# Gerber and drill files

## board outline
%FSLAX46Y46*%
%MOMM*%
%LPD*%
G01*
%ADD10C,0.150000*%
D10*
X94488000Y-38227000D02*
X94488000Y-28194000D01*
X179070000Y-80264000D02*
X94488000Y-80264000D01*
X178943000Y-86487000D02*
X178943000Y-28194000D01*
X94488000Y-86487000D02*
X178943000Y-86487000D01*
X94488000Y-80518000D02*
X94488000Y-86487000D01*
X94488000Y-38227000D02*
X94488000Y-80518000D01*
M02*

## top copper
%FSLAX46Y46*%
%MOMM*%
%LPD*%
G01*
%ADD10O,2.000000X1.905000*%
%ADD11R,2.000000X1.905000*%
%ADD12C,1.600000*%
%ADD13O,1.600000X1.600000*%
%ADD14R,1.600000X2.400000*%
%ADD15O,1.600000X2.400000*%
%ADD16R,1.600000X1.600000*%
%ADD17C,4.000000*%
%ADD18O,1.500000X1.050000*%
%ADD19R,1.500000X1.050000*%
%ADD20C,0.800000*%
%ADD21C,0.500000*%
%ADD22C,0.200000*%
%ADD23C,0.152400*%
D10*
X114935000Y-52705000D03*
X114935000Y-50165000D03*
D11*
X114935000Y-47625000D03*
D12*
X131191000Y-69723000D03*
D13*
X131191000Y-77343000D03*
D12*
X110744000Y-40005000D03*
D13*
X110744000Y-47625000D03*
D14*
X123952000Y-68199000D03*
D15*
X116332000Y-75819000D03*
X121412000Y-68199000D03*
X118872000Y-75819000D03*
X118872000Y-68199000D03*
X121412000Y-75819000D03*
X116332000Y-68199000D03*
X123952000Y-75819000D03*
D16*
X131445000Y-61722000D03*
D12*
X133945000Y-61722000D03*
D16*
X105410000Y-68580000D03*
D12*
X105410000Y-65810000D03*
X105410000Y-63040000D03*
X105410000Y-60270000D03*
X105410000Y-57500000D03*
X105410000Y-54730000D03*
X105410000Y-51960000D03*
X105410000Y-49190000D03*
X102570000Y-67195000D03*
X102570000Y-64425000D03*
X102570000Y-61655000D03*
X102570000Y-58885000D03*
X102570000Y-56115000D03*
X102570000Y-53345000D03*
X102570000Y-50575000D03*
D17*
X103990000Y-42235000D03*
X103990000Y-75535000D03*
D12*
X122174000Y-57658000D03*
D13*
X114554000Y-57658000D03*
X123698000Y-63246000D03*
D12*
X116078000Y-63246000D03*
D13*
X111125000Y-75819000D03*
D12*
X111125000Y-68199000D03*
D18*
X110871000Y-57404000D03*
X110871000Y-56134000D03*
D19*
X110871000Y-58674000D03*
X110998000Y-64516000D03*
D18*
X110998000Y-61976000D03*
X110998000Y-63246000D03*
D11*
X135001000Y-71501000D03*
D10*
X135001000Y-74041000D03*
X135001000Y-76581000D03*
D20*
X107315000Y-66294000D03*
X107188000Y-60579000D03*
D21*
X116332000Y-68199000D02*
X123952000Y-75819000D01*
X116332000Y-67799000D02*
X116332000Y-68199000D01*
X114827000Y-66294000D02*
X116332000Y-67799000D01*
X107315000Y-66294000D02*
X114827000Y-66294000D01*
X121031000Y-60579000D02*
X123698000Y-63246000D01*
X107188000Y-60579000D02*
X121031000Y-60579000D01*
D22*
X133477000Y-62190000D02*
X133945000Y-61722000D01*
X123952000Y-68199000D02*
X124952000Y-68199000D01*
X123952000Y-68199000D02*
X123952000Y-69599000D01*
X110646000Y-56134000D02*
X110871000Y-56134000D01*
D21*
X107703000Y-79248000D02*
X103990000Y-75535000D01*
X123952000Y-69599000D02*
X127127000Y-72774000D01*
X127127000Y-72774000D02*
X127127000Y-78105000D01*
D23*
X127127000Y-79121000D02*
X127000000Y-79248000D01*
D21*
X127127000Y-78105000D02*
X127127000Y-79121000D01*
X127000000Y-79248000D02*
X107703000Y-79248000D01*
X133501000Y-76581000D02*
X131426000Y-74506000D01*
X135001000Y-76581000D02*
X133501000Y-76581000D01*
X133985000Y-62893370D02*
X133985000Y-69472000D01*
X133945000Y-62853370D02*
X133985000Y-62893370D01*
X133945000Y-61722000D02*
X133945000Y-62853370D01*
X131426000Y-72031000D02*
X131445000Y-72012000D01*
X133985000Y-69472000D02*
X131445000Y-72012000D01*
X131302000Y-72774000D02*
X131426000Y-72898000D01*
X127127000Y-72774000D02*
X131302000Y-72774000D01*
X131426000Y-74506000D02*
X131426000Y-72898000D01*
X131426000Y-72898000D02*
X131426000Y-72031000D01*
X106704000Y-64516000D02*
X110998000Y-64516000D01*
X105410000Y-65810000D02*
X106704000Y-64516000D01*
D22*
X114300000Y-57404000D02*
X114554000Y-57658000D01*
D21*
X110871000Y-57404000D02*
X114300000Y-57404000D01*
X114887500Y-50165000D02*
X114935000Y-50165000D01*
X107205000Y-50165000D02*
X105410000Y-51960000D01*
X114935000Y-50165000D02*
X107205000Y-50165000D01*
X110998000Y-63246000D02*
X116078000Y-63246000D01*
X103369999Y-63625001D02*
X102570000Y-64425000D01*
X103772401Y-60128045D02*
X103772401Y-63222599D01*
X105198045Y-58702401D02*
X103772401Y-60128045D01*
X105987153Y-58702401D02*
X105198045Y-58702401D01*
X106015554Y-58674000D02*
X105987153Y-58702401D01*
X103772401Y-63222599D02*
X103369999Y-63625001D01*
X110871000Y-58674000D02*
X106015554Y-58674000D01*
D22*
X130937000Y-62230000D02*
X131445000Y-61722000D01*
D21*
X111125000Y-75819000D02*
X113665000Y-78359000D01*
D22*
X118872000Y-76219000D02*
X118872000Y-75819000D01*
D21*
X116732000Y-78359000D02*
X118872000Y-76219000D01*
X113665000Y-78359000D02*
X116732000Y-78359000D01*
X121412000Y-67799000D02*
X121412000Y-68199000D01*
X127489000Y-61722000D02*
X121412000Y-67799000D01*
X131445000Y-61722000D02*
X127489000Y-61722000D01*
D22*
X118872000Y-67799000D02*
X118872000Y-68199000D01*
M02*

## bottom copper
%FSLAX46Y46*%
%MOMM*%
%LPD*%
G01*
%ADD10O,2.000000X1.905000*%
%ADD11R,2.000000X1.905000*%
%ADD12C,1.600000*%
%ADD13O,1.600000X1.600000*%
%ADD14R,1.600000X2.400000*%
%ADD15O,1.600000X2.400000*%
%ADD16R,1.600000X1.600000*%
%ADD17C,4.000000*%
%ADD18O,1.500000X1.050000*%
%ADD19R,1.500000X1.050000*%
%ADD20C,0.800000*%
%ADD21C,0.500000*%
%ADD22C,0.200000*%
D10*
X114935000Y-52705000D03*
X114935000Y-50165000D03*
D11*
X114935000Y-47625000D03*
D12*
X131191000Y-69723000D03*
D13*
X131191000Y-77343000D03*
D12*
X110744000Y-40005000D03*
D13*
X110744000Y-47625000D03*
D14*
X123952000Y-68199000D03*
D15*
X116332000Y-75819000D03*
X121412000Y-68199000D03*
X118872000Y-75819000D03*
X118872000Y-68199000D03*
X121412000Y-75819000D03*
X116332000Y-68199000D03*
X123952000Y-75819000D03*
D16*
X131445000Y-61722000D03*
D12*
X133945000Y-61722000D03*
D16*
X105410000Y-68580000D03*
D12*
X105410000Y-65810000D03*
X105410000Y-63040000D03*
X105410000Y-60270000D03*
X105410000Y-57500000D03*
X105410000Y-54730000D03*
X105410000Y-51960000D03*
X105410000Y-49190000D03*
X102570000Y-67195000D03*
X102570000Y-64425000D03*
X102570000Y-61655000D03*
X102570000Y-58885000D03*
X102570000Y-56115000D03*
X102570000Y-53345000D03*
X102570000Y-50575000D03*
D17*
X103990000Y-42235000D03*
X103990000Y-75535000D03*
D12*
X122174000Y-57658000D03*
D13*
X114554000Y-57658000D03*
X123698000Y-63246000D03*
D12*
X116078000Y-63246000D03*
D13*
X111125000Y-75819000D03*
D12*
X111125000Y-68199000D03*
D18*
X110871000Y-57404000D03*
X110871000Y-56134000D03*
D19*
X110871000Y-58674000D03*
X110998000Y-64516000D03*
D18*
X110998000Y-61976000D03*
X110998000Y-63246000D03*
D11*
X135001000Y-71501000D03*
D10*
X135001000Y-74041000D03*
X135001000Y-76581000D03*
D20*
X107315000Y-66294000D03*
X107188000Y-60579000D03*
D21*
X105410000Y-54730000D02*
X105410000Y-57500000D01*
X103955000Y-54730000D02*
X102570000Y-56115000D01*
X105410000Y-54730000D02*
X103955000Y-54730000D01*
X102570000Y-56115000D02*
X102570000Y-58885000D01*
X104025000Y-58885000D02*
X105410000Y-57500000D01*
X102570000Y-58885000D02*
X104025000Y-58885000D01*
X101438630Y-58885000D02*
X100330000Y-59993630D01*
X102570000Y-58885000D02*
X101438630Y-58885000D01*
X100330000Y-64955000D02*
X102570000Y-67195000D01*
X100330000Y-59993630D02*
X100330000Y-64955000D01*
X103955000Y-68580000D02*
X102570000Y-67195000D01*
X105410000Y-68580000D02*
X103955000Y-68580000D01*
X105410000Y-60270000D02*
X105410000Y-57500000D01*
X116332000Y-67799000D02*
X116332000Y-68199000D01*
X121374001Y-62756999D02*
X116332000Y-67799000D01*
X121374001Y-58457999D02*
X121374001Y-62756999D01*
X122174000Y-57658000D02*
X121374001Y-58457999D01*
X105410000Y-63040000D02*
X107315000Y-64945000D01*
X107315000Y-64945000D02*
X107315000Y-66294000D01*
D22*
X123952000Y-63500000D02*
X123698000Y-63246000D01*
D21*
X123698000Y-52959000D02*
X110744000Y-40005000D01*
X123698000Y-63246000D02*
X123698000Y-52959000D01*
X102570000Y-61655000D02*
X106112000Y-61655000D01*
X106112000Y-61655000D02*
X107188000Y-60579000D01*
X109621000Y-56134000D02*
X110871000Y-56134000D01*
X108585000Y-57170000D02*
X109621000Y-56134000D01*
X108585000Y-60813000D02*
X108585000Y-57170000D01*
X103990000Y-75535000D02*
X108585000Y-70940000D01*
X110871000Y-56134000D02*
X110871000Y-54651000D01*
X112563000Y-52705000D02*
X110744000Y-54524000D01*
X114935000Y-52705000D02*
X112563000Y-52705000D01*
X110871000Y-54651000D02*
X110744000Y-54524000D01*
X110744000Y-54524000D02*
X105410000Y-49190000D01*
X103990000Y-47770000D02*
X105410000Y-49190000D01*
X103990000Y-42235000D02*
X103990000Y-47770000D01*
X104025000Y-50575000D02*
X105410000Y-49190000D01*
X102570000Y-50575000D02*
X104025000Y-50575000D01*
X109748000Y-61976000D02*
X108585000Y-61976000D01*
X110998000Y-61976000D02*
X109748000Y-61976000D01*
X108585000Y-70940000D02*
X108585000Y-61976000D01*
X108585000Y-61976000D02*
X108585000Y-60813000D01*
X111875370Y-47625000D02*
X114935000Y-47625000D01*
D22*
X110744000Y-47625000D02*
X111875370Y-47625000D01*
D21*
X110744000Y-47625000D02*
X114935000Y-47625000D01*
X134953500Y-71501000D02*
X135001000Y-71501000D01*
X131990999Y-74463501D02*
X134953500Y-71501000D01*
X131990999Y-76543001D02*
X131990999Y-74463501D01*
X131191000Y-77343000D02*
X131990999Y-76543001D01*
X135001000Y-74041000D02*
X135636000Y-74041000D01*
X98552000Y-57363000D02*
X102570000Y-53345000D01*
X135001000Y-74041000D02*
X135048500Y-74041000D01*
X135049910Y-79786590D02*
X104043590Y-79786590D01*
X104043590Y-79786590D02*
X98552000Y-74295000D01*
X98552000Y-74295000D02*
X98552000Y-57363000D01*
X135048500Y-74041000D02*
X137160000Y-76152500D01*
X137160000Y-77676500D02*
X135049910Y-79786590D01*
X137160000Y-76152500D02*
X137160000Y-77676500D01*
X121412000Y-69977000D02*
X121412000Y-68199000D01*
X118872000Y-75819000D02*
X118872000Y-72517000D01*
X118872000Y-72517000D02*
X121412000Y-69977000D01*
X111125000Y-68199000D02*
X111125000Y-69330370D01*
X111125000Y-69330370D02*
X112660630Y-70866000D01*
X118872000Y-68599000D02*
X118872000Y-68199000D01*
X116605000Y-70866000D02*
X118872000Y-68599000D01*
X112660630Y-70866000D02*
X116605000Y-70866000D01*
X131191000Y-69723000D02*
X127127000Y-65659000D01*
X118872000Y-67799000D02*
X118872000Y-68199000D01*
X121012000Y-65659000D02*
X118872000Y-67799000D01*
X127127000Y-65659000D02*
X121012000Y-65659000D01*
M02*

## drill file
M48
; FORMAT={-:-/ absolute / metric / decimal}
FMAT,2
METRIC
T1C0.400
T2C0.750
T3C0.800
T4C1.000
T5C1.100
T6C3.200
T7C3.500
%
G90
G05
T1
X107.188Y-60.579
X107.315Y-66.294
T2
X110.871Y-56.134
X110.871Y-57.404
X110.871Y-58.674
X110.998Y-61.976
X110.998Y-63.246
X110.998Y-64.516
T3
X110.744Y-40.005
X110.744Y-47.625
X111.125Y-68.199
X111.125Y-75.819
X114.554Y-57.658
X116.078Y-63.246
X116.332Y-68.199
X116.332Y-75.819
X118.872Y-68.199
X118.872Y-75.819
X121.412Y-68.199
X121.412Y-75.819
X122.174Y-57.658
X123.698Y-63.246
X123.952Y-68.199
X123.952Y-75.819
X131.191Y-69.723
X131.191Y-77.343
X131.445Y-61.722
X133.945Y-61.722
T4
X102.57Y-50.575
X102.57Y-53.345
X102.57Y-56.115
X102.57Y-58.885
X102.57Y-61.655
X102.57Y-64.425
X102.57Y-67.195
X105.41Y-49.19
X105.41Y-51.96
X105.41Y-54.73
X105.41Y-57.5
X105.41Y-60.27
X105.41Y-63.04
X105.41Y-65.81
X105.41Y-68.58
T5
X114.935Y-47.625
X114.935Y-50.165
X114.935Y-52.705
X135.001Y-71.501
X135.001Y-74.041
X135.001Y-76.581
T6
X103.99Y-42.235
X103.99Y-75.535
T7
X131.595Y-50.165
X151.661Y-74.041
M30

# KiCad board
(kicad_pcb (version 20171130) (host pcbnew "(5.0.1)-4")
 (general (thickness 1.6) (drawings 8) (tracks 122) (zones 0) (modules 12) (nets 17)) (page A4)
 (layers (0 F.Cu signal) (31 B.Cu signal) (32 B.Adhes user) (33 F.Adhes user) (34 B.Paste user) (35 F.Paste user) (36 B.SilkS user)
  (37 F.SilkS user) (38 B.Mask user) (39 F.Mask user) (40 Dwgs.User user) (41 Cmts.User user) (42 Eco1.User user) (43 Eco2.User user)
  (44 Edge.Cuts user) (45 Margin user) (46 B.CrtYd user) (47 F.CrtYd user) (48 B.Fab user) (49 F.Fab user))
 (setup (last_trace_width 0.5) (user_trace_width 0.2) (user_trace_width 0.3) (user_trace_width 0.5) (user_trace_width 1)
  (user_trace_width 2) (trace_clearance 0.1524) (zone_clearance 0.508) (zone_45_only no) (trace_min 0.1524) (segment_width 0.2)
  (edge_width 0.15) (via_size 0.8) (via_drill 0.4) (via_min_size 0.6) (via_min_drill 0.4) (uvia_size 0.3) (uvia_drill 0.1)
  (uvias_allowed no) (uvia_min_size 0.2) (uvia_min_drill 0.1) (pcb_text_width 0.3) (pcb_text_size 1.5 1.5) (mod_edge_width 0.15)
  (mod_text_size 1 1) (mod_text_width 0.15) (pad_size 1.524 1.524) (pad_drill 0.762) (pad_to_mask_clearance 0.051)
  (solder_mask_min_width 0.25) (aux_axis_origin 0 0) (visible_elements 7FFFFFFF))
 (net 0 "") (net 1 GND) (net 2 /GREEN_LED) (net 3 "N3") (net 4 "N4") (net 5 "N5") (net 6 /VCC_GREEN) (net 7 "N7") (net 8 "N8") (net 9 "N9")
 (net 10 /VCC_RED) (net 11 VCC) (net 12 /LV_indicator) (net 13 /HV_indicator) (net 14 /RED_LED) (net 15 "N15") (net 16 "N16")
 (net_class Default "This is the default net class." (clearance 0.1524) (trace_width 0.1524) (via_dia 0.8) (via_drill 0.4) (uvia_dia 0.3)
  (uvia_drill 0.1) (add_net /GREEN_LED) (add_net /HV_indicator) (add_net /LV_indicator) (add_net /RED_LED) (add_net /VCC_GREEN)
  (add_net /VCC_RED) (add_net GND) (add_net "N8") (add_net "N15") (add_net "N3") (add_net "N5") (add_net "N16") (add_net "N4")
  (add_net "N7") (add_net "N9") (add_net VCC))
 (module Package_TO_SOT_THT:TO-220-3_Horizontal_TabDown (layer F.Cu) (at 114.935 47.625 270)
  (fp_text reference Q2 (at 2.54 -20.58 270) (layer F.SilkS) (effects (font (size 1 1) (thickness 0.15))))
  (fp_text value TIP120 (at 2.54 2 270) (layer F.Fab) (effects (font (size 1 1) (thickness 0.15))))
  (pad 3 thru_hole oval (at 5.08 0 270) (size 1.905 2) (drill 1.1) (layers *.Cu *.Mask) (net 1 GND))
  (pad 2 thru_hole oval (at 2.54 0 270) (size 1.905 2) (drill 1.1) (layers *.Cu *.Mask) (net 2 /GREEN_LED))
  (pad 1 thru_hole rect (at 0 0 270) (size 1.905 2) (drill 1.1) (layers *.Cu *.Mask) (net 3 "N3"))
  (pad "" np_thru_hole oval (at 2.54 -16.66 270) (size 3.5 3.5) (drill 3.5) (layers *.Cu *.Mask)))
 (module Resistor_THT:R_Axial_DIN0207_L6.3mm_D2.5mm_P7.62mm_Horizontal (layer F.Cu) (at 131.191 69.723 270)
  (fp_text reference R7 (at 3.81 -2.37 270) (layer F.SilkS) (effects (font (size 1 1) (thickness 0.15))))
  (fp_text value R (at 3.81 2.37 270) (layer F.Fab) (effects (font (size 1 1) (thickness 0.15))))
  (pad 1 thru_hole circle (at 0 0 270) (size 1.6 1.6) (drill 0.8) (layers *.Cu *.Mask) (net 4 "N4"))
  (pad 2 thru_hole oval (at 7.62 0 270) (size 1.6 1.6) (drill 0.8) (layers *.Cu *.Mask) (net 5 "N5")))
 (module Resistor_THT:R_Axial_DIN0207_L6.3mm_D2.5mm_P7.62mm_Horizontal (layer F.Cu) (at 110.744 40.005 270)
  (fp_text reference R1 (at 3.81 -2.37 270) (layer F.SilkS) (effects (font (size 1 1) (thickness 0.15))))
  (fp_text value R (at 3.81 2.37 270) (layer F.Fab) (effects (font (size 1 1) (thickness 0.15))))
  (pad 1 thru_hole circle (at 0 0 270) (size 1.6 1.6) (drill 0.8) (layers *.Cu *.Mask) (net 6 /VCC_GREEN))
  (pad 2 thru_hole oval (at 7.62 0 270) (size 1.6 1.6) (drill 0.8) (layers *.Cu *.Mask) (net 3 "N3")))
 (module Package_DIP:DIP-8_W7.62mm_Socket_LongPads (layer F.Cu) (at 123.952 68.199 270)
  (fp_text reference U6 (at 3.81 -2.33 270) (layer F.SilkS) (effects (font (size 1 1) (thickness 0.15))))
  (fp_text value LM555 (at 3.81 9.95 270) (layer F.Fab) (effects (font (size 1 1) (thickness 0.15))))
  (pad 1 thru_hole rect (at 0 0 270) (size 2.4 1.6) (drill 0.8) (layers *.Cu *.Mask) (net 1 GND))
  (pad 5 thru_hole oval (at 7.62 7.62 270) (size 2.4 1.6) (drill 0.8) (layers *.Cu *.Mask) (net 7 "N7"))
  (pad 2 thru_hole oval (at 0 2.54 270) (size 2.4 1.6) (drill 0.8) (layers *.Cu *.Mask) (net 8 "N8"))
  (pad 6 thru_hole oval (at 7.62 5.08 270) (size 2.4 1.6) (drill 0.8) (layers *.Cu *.Mask) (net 8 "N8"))
  (pad 3 thru_hole oval (at 0 5.08 270) (size 2.4 1.6) (drill 0.8) (layers *.Cu *.Mask) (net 4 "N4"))
  (pad 7 thru_hole oval (at 7.62 2.54 270) (size 2.4 1.6) (drill 0.8) (layers *.Cu *.Mask) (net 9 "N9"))
  (pad 4 thru_hole oval (at 0 7.62 270) (size 2.4 1.6) (drill 0.8) (layers *.Cu *.Mask) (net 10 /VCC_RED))
  (pad 8 thru_hole oval (at 7.62 0 270) (size 2.4 1.6) (drill 0.8) (layers *.Cu *.Mask) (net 10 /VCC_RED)))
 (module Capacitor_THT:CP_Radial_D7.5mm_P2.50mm (layer F.Cu) (at 131.445 61.722)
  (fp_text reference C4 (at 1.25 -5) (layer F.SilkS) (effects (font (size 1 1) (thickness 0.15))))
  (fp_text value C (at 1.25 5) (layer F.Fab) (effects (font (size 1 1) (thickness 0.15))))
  (pad 1 thru_hole rect (at 0 0) (size 1.6 1.6) (drill 0.8) (layers *.Cu *.Mask) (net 8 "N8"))
  (pad 2 thru_hole circle (at 2.5 0) (size 1.6 1.6) (drill 0.8) (layers *.Cu *.Mask) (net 1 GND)))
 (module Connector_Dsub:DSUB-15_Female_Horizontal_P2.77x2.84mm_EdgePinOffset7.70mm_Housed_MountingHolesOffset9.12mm (layer F.Cu)
  (at 105.41 68.58 270)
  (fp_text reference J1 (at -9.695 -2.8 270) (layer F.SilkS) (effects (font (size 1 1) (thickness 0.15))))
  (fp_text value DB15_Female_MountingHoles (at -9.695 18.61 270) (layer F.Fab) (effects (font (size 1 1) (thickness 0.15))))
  (pad 1 thru_hole rect (at 0 0 270) (size 1.6 1.6) (drill 1) (layers *.Cu *.Mask) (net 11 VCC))
  (pad 2 thru_hole circle (at -2.77 0 270) (size 1.6 1.6) (drill 1) (layers *.Cu *.Mask) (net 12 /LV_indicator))
  (pad 3 thru_hole circle (at -5.54 0 270) (size 1.6 1.6) (drill 1) (layers *.Cu *.Mask) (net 10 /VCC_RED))
  (pad 4 thru_hole circle (at -8.31 0 270) (size 1.6 1.6) (drill 1) (layers *.Cu *.Mask) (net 11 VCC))
  (pad 5 thru_hole circle (at -11.08 0 270) (size 1.6 1.6) (drill 1) (layers *.Cu *.Mask) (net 11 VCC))
  (pad 6 thru_hole circle (at -13.85 0 270) (size 1.6 1.6) (drill 1) (layers *.Cu *.Mask) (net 11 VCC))
  (pad 7 thru_hole circle (at -16.62 0 270) (size 1.6 1.6) (drill 1) (layers *.Cu *.Mask) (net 2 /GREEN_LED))
  (pad 8 thru_hole circle (at -19.39 0 270) (size 1.6 1.6) (drill 1) (layers *.Cu *.Mask) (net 1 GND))
  (pad 9 thru_hole circle (at -1.385 2.84 270) (size 1.6 1.6) (drill 1) (layers *.Cu *.Mask) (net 11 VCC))
  (pad 10 thru_hole circle (at -4.155 2.84 270) (size 1.6 1.6) (drill 1) (layers *.Cu *.Mask) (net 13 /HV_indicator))
  (pad 11 thru_hole circle (at -6.925 2.84 270) (size 1.6 1.6) (drill 1) (layers *.Cu *.Mask) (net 6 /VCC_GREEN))
  (pad 12 thru_hole circle (at -9.695 2.84 270) (size 1.6 1.6) (drill 1) (layers *.Cu *.Mask) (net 11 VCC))
  (pad 13 thru_hole circle (at -12.465 2.84 270) (size 1.6 1.6) (drill 1) (layers *.Cu *.Mask) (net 11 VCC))
  (pad 14 thru_hole circle (at -15.235 2.84 270) (size 1.6 1.6) (drill 1) (layers *.Cu *.Mask) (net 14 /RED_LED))
  (pad 15 thru_hole circle (at -18.005 2.84 270) (size 1.6 1.6) (drill 1) (layers *.Cu *.Mask) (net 1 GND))
  (pad 0 thru_hole circle (at -26.345 1.42 270) (size 4 4) (drill 3.2) (layers *.Cu *.Mask) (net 1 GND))
  (pad 0 thru_hole circle (at 6.955 1.42 270) (size 4 4) (drill 3.2) (layers *.Cu *.Mask) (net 1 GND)))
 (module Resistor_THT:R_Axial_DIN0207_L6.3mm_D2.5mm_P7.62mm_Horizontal (layer F.Cu) (at 122.174 57.658 180)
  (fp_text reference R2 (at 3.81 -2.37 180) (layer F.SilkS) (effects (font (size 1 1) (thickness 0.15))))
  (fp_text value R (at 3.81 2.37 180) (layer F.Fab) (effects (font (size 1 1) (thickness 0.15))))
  (pad 1 thru_hole circle (at 0 0 180) (size 1.6 1.6) (drill 0.8) (layers *.Cu *.Mask) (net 10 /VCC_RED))
  (pad 2 thru_hole oval (at 7.62 0 180) (size 1.6 1.6) (drill 0.8) (layers *.Cu *.Mask) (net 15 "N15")))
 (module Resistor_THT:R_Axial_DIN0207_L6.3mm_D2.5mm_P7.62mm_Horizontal (layer F.Cu) (at 116.078 63.246)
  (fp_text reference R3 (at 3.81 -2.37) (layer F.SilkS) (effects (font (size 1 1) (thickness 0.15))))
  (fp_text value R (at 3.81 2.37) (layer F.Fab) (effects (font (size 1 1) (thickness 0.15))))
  (pad 2 thru_hole oval (at 7.62 0) (size 1.6 1.6) (drill 0.8) (layers *.Cu *.Mask) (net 6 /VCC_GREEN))
  (pad 1 thru_hole circle (at 0 0) (size 1.6 1.6) (drill 0.8) (layers *.Cu *.Mask) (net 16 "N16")))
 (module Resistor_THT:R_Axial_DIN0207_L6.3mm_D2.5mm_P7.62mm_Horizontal (layer F.Cu) (at 111.125 68.199 270)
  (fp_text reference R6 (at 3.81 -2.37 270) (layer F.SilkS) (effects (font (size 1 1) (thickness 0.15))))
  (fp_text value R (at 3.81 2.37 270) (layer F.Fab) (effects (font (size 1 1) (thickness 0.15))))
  (pad 2 thru_hole oval (at 7.62 0 270) (size 1.6 1.6) (drill 0.8) (layers *.Cu *.Mask) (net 8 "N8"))
  (pad 1 thru_hole circle (at 0 0 270) (size 1.6 1.6) (drill 0.8) (layers *.Cu *.Mask) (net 4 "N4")))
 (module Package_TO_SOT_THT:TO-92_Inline (layer F.Cu) (at 110.871 58.674 90)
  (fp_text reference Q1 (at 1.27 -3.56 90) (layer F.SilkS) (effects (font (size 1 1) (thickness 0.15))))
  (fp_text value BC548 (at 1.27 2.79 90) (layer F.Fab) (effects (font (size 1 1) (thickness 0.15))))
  (pad 2 thru_hole oval (at 1.27 0 90) (size 1.05 1.5) (drill 0.75) (layers *.Cu *.Mask) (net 15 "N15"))
  (pad 3 thru_hole oval (at 2.54 0 90) (size 1.05 1.5) (drill 0.75) (layers *.Cu *.Mask) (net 1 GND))
  (pad 1 thru_hole rect (at 0 0 90) (size 1.05 1.5) (drill 0.75) (layers *.Cu *.Mask) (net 13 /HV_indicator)))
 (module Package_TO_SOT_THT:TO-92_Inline (layer F.Cu) (at 110.998 64.516 90)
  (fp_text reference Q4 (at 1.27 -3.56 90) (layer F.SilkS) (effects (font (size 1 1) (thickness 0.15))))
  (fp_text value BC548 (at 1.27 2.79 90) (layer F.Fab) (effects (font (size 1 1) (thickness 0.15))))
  (pad 1 thru_hole rect (at 0 0 90) (size 1.05 1.5) (drill 0.75) (layers *.Cu *.Mask) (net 12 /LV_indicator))
  (pad 3 thru_hole oval (at 2.54 0 90) (size 1.05 1.5) (drill 0.75) (layers *.Cu *.Mask) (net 1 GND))
  (pad 2 thru_hole oval (at 1.27 0 90) (size 1.05 1.5) (drill 0.75) (layers *.Cu *.Mask) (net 16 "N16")))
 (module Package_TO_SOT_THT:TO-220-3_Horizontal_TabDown (layer F.Cu) (at 135.001 71.501 270)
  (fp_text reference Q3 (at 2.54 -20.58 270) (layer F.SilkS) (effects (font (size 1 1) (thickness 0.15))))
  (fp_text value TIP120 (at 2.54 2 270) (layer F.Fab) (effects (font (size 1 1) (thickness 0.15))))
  (pad "" np_thru_hole oval (at 2.54 -16.66 270) (size 3.5 3.5) (drill 3.5) (layers *.Cu *.Mask))
  (pad 1 thru_hole rect (at 0 0 270) (size 1.905 2) (drill 1.1) (layers *.Cu *.Mask) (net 5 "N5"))
  (pad 2 thru_hole oval (at 2.54 0 270) (size 1.905 2) (drill 1.1) (layers *.Cu *.Mask) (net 14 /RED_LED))
  (pad 3 thru_hole oval (at 5.08 0 270) (size 1.905 2) (drill 1.1) (layers *.Cu *.Mask) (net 1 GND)))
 (gr_line (start 94.488 38.227) (end 94.488 28.194) (layer Edge.Cuts) (width 0.15))
 (gr_line (start 179.07 80.264) (end 94.488 80.264) (layer Edge.Cuts) (width 0.15))
 (gr_line (start 178.943 86.487) (end 178.943 28.194) (layer Edge.Cuts) (width 0.15))
 (gr_line (start 94.488 86.487) (end 178.943 86.487) (layer Edge.Cuts) (width 0.15))
 (gr_line (start 94.488 80.518) (end 94.488 86.487) (layer Edge.Cuts) (width 0.15))
 (gr_line (start 94.488 38.227) (end 94.488 80.518) (layer Edge.Cuts) (width 0.15))
 (segment (start 105.41 54.73) (end 105.41 57.5) (width 0.5) (layer B.Cu) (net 11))
 (segment (start 103.955 54.73) (end 102.57 56.115) (width 0.5) (layer B.Cu) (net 11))
 (segment (start 105.41 54.73) (end 103.955 54.73) (width 0.5) (layer B.Cu) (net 11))
 (segment (start 102.57 56.115) (end 102.57 58.885) (width 0.5) (layer B.Cu) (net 11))
 (segment (start 104.025 58.885) (end 105.41 57.5) (width 0.5) (layer B.Cu) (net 11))
 (segment (start 102.57 58.885) (end 104.025 58.885) (width 0.5) (layer B.Cu) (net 11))
 (segment (start 101.43863 58.885) (end 100.33 59.99363) (width 0.5) (layer B.Cu) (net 11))
 (segment (start 102.57 58.885) (end 101.43863 58.885) (width 0.5) (layer B.Cu) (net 11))
 (segment (start 100.33 64.955) (end 102.57 67.195) (width 0.5) (layer B.Cu) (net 11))
 (segment (start 100.33 59.99363) (end 100.33 64.955) (width 0.5) (layer B.Cu) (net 11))
 (segment (start 103.955 68.58) (end 102.57 67.195) (width 0.5) (layer B.Cu) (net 11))
 (segment (start 105.41 68.58) (end 103.955 68.58) (width 0.5) (layer B.Cu) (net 11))
 (segment (start 105.41 60.27) (end 105.41 57.5) (width 0.5) (layer B.Cu) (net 11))
 (segment (start 116.332 68.199) (end 123.952 75.819) (width 0.5) (layer F.Cu) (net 10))
 (segment (start 116.332 67.799) (end 116.332 68.199) (width 0.5) (layer B.Cu) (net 10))
 (segment (start 121.374001 62.756999) (end 116.332 67.799) (width 0.5) (layer B.Cu) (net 10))
 (segment (start 121.374001 58.457999) (end 121.374001 62.756999) (width 0.5) (layer B.Cu) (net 10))
 (segment (start 122.174 57.658) (end 121.374001 58.457999) (width 0.5) (layer B.Cu) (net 10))
 (segment (start 105.41 63.04) (end 107.315 64.945) (width 0.5) (layer B.Cu) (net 10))
 (via (at 107.315 66.294) (size 0.8) (drill 0.4) (layers F.Cu B.Cu) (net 10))
 (segment (start 107.315 64.945) (end 107.315 66.294) (width 0.5) (layer B.Cu) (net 10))
 (segment (start 116.332 67.799) (end 116.332 68.199) (width 0.5) (layer F.Cu) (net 10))
 (segment (start 114.827 66.294) (end 116.332 67.799) (width 0.5) (layer F.Cu) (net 10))
 (segment (start 107.315 66.294) (end 114.827 66.294) (width 0.5) (layer F.Cu) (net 10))
 (segment (start 123.952 63.5) (end 123.698 63.246) (width 0.2) (layer B.Cu) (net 6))
 (segment (start 123.698 52.959) (end 110.744 40.005) (width 0.5) (layer B.Cu) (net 6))
 (segment (start 123.698 63.246) (end 123.698 52.959) (width 0.5) (layer B.Cu) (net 6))
 (segment (start 102.57 61.655) (end 106.112 61.655) (width 0.5) (layer B.Cu) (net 6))
 (via (at 107.188 60.579) (size 0.8) (drill 0.4) (layers F.Cu B.Cu) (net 6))
 (segment (start 106.112 61.655) (end 107.188 60.579) (width 0.5) (layer B.Cu) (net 6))
 (segment (start 121.031 60.579) (end 123.698 63.246) (width 0.5) (layer F.Cu) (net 6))
 (segment (start 107.188 60.579) (end 121.031 60.579) (width 0.5) (layer F.Cu) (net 6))
 (segment (start 133.477 62.19) (end 133.945 61.722) (width 0.2) (layer F.Cu) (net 1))
 (segment (start 123.952 68.199) (end 124.952 68.199) (width 0.2) (layer F.Cu) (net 1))
 (segment (start 123.952 68.199) (end 123.952 69.599) (width 0.2) (layer F.Cu) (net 1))
 (segment (start 110.646 56.134) (end 110.871 56.134) (width 0.2) (layer F.Cu) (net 1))
 (segment (start 109.621 56.134) (end 110.871 56.134) (width 0.5) (layer B.Cu) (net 1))
 (segment (start 108.585 57.17) (end 109.621 56.134) (width 0.5) (layer B.Cu) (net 1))
 (segment (start 108.585 60.813) (end 108.585 57.17) (width 0.5) (layer B.Cu) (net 1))
 (segment (start 103.99 75.535) (end 108.585 70.94) (width 0.5) (layer B.Cu) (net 1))
 (segment (start 110.871 56.134) (end 110.871 54.651) (width 0.5) (layer B.Cu) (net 1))
 (segment (start 107.703 79.248) (end 103.99 75.535) (width 0.5) (layer F.Cu) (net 1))
 (segment (start 123.952 69.599) (end 127.127 72.774) (width 0.5) (layer F.Cu) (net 1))
 (segment (start 127.127 72.774) (end 127.127 78.105) (width 0.5) (layer F.Cu) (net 1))
 (segment (start 127.127 79.121) (end 127 79.248) (width 0.1524) (layer F.Cu) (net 1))
 (segment (start 127.127 78.105) (end 127.127 79.121) (width 0.5) (layer F.Cu) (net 1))
 (segment (start 127 79.248) (end 107.703 79.248) (width 0.5) (layer F.Cu) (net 1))
 (segment (start 133.501 76.581) (end 131.426 74.506) (width 0.5) (layer F.Cu) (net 1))
 (segment (start 135.001 76.581) (end 133.501 76.581) (width 0.5) (layer F.Cu) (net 1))
 (segment (start 133.985 62.89337) (end 133.985 69.472) (width 0.5) (layer F.Cu) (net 1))
 (segment (start 133.945 62.85337) (end 133.985 62.89337) (width 0.5) (layer F.Cu) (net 1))
 (segment (start 133.945 61.722) (end 133.945 62.85337) (width 0.5) (layer F.Cu) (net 1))
 (segment (start 131.426 72.031) (end 131.445 72.012) (width 0.5) (layer F.Cu) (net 1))
 (segment (start 133.985 69.472) (end 131.445 72.012) (width 0.5) (layer F.Cu) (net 1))
 (segment (start 131.302 72.774) (end 131.426 72.898) (width 0.5) (layer F.Cu) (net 1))
 (segment (start 127.127 72.774) (end 131.302 72.774) (width 0.5) (layer F.Cu) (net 1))
 (segment (start 131.426 74.506) (end 131.426 72.898) (width 0.5) (layer F.Cu) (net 1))
 (segment (start 131.426 72.898) (end 131.426 72.031) (width 0.5) (layer F.Cu) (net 1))
 (segment (start 112.563 52.705) (end 110.744 54.524) (width 0.5) (layer B.Cu) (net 1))
 (segment (start 114.935 52.705) (end 112.563 52.705) (width 0.5) (layer B.Cu) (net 1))
 (segment (start 110.871 54.651) (end 110.744 54.524) (width 0.5) (layer B.Cu) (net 1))
 (segment (start 110.744 54.524) (end 105.41 49.19) (width 0.5) (layer B.Cu) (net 1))
 (segment (start 103.99 47.77) (end 105.41 49.19) (width 0.5) (layer B.Cu) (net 1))
 (segment (start 103.99 42.235) (end 103.99 47.77) (width 0.5) (layer B.Cu) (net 1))
 (segment (start 104.025 50.575) (end 105.41 49.19) (width 0.5) (layer B.Cu) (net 1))
 (segment (start 102.57 50.575) (end 104.025 50.575) (width 0.5) (layer B.Cu) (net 1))
 (segment (start 109.748 61.976) (end 108.585 61.976) (width 0.5) (layer B.Cu) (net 1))
 (segment (start 110.998 61.976) (end 109.748 61.976) (width 0.5) (layer B.Cu) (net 1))
 (segment (start 108.585 70.94) (end 108.585 61.976) (width 0.5) (layer B.Cu) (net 1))
 (segment (start 108.585 61.976) (end 108.585 60.813) (width 0.5) (layer B.Cu) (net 1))
 (segment (start 106.704 64.516) (end 110.998 64.516) (width 0.5) (layer F.Cu) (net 12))
 (segment (start 105.41 65.81) (end 106.704 64.516) (width 0.5) (layer F.Cu) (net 12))
 (segment (start 114.3 57.404) (end 114.554 57.658) (width 0.2) (layer F.Cu) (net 15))
 (segment (start 110.871 57.404) (end 114.3 57.404) (width 0.5) (layer F.Cu) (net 15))
 (segment (start 114.8875 50.165) (end 114.935 50.165) (width 0.5) (layer F.Cu) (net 2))
 (segment (start 107.205 50.165) (end 105.41 51.96) (width 0.5) (layer F.Cu) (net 2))
 (segment (start 114.935 50.165) (end 107.205 50.165) (width 0.5) (layer F.Cu) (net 2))
 (segment (start 111.87537 47.625) (end 114.935 47.625) (width 0.5) (layer B.Cu) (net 3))
 (segment (start 110.744 47.625) (end 111.87537 47.625) (width 0.2) (layer B.Cu) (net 3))
 (segment (start 110.744 47.625) (end 114.935 47.625) (width 0.5) (layer B.Cu) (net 3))
 (segment (start 134.9535 71.501) (end 135.001 71.501) (width 0.5) (layer B.Cu) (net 5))
 (segment (start 131.990999 74.463501) (end 134.9535 71.501) (width 0.5) (layer B.Cu) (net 5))
 (segment (start 131.990999 76.543001) (end 131.990999 74.463501) (width 0.5) (layer B.Cu) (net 5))
 (segment (start 131.191 77.343) (end 131.990999 76.543001) (width 0.5) (layer B.Cu) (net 5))
 (segment (start 135.001 74.041) (end 135.636 74.041) (width 0.5) (layer B.Cu) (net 14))
 (segment (start 98.552 57.363) (end 102.57 53.345) (width 0.5) (layer B.Cu) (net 14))
 (segment (start 135.001 74.041) (end 135.0485 74.041) (width 0.5) (layer B.Cu) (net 14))
 (segment (start 135.04991 79.78659) (end 104.04359 79.78659) (width 0.5) (layer B.Cu) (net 14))
 (segment (start 104.04359 79.78659) (end 98.552 74.295) (width 0.5) (layer B.Cu) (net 14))
 (segment (start 98.552 74.295) (end 98.552 57.363) (width 0.5) (layer B.Cu) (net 14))
 (segment (start 135.0485 74.041) (end 137.16 76.1525) (width 0.5) (layer B.Cu) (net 14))
 (segment (start 137.16 77.6765) (end 135.04991 79.78659) (width 0.5) (layer B.Cu) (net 14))
 (segment (start 137.16 76.1525) (end 137.16 77.6765) (width 0.5) (layer B.Cu) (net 14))
 (segment (start 110.998 63.246) (end 116.078 63.246) (width 0.5) (layer F.Cu) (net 16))
 (segment (start 103.369999 63.625001) (end 102.57 64.425) (width 0.5) (layer F.Cu) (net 13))
 (segment (start 103.772401 60.128045) (end 103.772401 63.222599) (width 0.5) (layer F.Cu) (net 13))
 (segment (start 105.198045 58.702401) (end 103.772401 60.128045) (width 0.5) (layer F.Cu) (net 13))
 (segment (start 105.987153 58.702401) (end 105.198045 58.702401) (width 0.5) (layer F.Cu) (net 13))
 (segment (start 106.015554 58.674) (end 105.987153 58.702401) (width 0.5) (layer F.Cu) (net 13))
 (segment (start 103.772401 63.222599) (end 103.369999 63.625001) (width 0.5) (layer F.Cu) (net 13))
 (segment (start 110.871 58.674) (end 106.015554 58.674) (width 0.5) (layer F.Cu) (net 13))
 (segment (start 130.937 62.23) (end 131.445 61.722) (width 0.2) (layer F.Cu) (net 8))
 (segment (start 111.125 75.819) (end 113.665 78.359) (width 0.5) (layer F.Cu) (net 8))
 (segment (start 118.872 76.219) (end 118.872 75.819) (width 0.2) (layer F.Cu) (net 8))
 (segment (start 116.732 78.359) (end 118.872 76.219) (width 0.5) (layer F.Cu) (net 8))
 (segment (start 113.665 78.359) (end 116.732 78.359) (width 0.5) (layer F.Cu) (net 8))
 (segment (start 121.412 67.799) (end 121.412 68.199) (width 0.5) (layer F.Cu) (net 8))
 (segment (start 127.489 61.722) (end 121.412 67.799) (width 0.5) (layer F.Cu) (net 8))
 (segment (start 131.445 61.722) (end 127.489 61.722) (width 0.5) (layer F.Cu) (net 8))
 (segment (start 121.412 69.977) (end 121.412 68.199) (width 0.5) (layer B.Cu) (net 8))
 (segment (start 118.872 75.819) (end 118.872 72.517) (width 0.5) (layer B.Cu) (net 8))
 (segment (start 118.872 72.517) (end 121.412 69.977) (width 0.5) (layer B.Cu) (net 8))
 (segment (start 118.872 67.799) (end 118.872 68.199) (width 0.2) (layer F.Cu) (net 4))
 (segment (start 111.125 68.199) (end 111.125 69.33037) (width 0.5) (layer B.Cu) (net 4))
 (segment (start 111.125 69.33037) (end 112.66063 70.866) (width 0.5) (layer B.Cu) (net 4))
 (segment (start 118.872 68.599) (end 118.872 68.199) (width 0.5) (layer B.Cu) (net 4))
 (segment (start 116.605 70.866) (end 118.872 68.599) (width 0.5) (layer B.Cu) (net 4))
 (segment (start 112.66063 70.866) (end 116.605 70.866) (width 0.5) (layer B.Cu) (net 4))
 (segment (start 131.191 69.723) (end 127.127 65.659) (width 0.5) (layer B.Cu) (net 4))
 (segment (start 118.872 67.799) (end 118.872 68.199) (width 0.5) (layer B.Cu) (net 4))
 (segment (start 121.012 65.659) (end 118.872 67.799) (width 0.5) (layer B.Cu) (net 4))
 (segment (start 127.127 65.659) (end 121.012 65.659) (width 0.5) (layer B.Cu) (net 4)))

